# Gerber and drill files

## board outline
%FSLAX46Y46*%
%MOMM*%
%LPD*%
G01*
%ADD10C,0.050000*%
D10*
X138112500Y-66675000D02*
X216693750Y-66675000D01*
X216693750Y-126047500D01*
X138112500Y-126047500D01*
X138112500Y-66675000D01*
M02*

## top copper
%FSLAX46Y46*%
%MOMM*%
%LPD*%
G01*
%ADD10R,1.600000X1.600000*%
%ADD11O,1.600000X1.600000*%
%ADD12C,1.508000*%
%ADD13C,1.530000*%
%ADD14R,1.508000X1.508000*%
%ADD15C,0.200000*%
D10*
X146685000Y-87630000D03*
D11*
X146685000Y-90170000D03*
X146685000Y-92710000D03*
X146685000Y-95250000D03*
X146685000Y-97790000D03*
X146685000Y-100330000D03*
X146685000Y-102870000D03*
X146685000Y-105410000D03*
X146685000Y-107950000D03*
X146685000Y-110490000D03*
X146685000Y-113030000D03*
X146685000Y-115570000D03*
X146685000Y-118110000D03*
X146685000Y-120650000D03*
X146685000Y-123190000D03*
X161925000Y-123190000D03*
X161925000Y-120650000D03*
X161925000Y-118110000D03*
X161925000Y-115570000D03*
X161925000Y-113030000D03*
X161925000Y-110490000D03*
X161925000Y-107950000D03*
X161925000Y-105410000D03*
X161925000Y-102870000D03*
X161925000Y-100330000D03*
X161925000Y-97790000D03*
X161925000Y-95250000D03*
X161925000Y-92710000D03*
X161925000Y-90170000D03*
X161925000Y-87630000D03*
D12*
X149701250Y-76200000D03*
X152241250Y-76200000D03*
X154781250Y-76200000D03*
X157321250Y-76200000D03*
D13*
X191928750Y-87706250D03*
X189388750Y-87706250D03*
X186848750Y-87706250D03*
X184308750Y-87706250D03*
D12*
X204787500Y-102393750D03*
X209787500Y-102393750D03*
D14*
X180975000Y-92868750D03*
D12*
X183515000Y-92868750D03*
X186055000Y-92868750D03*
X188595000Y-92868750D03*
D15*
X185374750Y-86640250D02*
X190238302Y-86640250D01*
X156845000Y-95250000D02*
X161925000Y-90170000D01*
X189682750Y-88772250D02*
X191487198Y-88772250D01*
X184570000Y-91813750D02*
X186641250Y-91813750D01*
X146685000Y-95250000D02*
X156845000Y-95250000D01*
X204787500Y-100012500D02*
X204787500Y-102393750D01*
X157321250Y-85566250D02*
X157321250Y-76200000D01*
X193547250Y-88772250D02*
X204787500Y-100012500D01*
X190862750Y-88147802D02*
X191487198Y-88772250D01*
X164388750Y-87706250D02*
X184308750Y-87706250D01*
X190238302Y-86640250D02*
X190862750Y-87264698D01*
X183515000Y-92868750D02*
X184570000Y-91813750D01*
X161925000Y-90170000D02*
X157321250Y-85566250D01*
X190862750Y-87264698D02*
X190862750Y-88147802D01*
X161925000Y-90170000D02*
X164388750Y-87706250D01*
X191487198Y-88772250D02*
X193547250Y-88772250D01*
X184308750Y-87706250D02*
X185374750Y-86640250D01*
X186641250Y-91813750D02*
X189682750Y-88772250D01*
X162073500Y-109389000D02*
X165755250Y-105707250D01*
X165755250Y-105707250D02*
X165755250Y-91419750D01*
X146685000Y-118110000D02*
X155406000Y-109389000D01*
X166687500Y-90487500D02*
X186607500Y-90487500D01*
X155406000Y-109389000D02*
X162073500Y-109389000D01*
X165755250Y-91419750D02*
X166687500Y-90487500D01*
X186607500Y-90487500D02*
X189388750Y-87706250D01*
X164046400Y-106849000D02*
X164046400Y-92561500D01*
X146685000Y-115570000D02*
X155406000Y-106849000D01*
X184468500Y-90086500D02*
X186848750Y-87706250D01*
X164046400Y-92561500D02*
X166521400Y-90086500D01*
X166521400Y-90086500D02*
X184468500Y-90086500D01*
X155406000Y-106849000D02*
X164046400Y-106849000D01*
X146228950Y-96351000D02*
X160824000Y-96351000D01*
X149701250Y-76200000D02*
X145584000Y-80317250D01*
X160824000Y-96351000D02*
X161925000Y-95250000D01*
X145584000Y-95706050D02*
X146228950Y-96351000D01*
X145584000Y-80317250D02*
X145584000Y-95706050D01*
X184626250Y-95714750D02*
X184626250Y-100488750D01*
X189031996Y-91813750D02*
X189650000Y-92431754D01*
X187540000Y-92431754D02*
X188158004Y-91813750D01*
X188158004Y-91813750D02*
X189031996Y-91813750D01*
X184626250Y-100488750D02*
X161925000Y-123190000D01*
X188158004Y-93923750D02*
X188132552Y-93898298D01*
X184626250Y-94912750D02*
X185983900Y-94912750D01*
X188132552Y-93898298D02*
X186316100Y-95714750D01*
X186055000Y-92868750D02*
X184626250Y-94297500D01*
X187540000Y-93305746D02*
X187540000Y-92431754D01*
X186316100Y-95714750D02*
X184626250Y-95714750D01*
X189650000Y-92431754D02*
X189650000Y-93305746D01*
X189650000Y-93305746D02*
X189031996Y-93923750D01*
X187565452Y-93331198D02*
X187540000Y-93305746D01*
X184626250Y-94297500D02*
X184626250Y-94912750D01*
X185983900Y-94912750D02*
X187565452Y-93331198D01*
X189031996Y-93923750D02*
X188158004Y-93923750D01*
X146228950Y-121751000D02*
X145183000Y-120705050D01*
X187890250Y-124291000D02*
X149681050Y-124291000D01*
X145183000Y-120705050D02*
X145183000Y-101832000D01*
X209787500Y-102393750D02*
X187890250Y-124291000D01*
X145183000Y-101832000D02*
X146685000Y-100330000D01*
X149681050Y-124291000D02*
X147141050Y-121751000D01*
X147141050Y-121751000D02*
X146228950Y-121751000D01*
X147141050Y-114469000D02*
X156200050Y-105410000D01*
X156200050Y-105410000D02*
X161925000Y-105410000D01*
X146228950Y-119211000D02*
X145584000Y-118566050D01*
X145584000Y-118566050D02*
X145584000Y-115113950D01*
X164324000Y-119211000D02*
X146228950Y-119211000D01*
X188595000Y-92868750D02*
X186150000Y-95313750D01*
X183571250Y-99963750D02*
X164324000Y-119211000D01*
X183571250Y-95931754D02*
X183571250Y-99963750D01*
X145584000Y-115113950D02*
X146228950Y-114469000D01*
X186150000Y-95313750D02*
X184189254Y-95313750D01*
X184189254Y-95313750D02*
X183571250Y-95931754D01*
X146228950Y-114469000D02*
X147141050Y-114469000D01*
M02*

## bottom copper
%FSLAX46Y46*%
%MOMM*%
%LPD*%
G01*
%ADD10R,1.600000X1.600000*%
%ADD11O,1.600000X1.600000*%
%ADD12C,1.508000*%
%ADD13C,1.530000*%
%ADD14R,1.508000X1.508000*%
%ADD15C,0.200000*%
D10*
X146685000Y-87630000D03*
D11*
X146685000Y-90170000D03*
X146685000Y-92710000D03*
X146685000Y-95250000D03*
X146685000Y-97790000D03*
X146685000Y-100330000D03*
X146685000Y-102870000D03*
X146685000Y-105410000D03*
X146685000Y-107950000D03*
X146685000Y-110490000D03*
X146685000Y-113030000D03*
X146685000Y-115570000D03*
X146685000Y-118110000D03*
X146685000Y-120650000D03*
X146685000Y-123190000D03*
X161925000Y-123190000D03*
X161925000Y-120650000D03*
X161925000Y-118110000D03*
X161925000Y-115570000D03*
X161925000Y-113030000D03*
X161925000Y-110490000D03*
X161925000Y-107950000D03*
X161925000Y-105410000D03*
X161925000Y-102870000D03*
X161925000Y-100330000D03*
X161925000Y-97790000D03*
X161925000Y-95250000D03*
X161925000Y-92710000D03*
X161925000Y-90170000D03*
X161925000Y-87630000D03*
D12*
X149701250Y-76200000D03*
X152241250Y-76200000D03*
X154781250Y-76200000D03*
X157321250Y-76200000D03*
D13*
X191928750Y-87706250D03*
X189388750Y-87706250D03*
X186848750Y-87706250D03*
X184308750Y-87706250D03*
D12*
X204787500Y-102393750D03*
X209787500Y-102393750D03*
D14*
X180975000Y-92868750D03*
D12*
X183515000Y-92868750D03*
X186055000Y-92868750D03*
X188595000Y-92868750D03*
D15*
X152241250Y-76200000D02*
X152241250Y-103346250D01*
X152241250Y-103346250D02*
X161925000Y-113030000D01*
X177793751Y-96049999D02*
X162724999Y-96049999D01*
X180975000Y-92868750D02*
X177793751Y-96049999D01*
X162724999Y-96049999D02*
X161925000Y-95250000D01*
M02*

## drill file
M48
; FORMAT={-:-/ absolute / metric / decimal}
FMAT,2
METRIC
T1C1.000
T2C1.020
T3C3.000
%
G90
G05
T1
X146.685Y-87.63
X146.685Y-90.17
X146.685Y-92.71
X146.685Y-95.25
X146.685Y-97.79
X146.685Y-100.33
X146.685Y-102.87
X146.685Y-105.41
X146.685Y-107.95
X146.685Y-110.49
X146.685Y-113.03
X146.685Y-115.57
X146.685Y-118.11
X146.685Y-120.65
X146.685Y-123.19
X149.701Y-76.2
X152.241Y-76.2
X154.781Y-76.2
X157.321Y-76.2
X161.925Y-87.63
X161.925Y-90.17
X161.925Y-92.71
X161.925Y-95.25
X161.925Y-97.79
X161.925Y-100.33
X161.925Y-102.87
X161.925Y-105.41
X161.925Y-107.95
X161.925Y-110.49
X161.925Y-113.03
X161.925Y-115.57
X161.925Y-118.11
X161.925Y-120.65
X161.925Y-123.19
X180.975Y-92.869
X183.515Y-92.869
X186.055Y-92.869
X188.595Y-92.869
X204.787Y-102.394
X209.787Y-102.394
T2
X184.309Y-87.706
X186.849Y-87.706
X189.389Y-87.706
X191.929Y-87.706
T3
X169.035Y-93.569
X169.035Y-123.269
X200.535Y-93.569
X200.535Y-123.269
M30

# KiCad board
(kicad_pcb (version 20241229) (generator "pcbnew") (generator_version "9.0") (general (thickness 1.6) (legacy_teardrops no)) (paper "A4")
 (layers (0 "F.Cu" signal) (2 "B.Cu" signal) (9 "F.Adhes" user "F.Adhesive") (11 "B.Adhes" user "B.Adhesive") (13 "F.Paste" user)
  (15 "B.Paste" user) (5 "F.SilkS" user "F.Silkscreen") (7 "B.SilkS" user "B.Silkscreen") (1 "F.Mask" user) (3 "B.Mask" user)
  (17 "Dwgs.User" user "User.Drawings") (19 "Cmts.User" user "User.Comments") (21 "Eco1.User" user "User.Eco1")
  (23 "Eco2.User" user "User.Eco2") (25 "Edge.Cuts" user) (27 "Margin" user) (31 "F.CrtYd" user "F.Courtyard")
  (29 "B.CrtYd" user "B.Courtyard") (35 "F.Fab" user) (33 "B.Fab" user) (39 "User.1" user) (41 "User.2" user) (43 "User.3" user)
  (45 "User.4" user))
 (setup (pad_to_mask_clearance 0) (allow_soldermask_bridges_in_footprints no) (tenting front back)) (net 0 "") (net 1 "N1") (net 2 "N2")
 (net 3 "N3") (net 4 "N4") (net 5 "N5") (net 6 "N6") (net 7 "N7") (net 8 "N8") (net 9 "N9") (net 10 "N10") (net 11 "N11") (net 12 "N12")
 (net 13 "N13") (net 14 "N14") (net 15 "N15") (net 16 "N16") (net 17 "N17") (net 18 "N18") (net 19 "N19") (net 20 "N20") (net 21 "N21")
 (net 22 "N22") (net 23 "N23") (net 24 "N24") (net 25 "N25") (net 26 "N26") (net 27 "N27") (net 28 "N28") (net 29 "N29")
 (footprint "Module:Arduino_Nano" (layer "F.Cu") (at 146.685 87.63)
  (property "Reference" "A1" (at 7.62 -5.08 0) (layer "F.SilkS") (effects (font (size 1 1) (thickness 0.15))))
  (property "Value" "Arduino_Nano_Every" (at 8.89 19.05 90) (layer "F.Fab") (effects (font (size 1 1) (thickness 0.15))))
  (pad "1" thru_hole rect (at 0 0) (size 1.6 1.6) (drill 1) (layers "*.Cu" "*.Mask") (remove_unused_layers no) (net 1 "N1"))
  (pad "2" thru_hole oval (at 0 2.54) (size 1.6 1.6) (drill 1) (layers "*.Cu" "*.Mask") (remove_unused_layers no) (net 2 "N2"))
  (pad "3" thru_hole oval (at 0 5.08) (size 1.6 1.6) (drill 1) (layers "*.Cu" "*.Mask") (remove_unused_layers no) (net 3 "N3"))
  (pad "4" thru_hole oval (at 0 7.62) (size 1.6 1.6) (drill 1) (layers "*.Cu" "*.Mask") (remove_unused_layers no) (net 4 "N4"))
  (pad "5" thru_hole oval (at 0 10.16) (size 1.6 1.6) (drill 1) (layers "*.Cu" "*.Mask") (remove_unused_layers no) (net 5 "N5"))
  (pad "6" thru_hole oval (at 0 12.7) (size 1.6 1.6) (drill 1) (layers "*.Cu" "*.Mask") (remove_unused_layers no) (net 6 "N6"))
  (pad "7" thru_hole oval (at 0 15.24) (size 1.6 1.6) (drill 1) (layers "*.Cu" "*.Mask") (remove_unused_layers no) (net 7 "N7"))
  (pad "8" thru_hole oval (at 0 17.78) (size 1.6 1.6) (drill 1) (layers "*.Cu" "*.Mask") (remove_unused_layers no) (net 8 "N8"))
  (pad "9" thru_hole oval (at 0 20.32) (size 1.6 1.6) (drill 1) (layers "*.Cu" "*.Mask") (remove_unused_layers no) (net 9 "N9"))
  (pad "10" thru_hole oval (at 0 22.86) (size 1.6 1.6) (drill 1) (layers "*.Cu" "*.Mask") (remove_unused_layers no) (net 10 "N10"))
  (pad "11" thru_hole oval (at 0 25.4) (size 1.6 1.6) (drill 1) (layers "*.Cu" "*.Mask") (remove_unused_layers no) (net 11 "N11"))
  (pad "12" thru_hole oval (at 0 27.94) (size 1.6 1.6) (drill 1) (layers "*.Cu" "*.Mask") (remove_unused_layers no) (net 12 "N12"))
  (pad "13" thru_hole oval (at 0 30.48) (size 1.6 1.6) (drill 1) (layers "*.Cu" "*.Mask") (remove_unused_layers no) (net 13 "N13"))
  (pad "14" thru_hole oval (at 0 33.02) (size 1.6 1.6) (drill 1) (layers "*.Cu" "*.Mask") (remove_unused_layers no) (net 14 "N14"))
  (pad "15" thru_hole oval (at 0 35.56) (size 1.6 1.6) (drill 1) (layers "*.Cu" "*.Mask") (remove_unused_layers no) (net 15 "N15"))
  (pad "16" thru_hole oval (at 15.24 35.56) (size 1.6 1.6) (drill 1) (layers "*.Cu" "*.Mask") (remove_unused_layers no) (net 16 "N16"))
  (pad "17" thru_hole oval (at 15.24 33.02) (size 1.6 1.6) (drill 1) (layers "*.Cu" "*.Mask") (remove_unused_layers no) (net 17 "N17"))
  (pad "18" thru_hole oval (at 15.24 30.48) (size 1.6 1.6) (drill 1) (layers "*.Cu" "*.Mask") (remove_unused_layers no) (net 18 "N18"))
  (pad "19" thru_hole oval (at 15.24 27.94) (size 1.6 1.6) (drill 1) (layers "*.Cu" "*.Mask") (remove_unused_layers no) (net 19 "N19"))
  (pad "20" thru_hole oval (at 15.24 25.4) (size 1.6 1.6) (drill 1) (layers "*.Cu" "*.Mask") (remove_unused_layers no) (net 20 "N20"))
  (pad "21" thru_hole oval (at 15.24 22.86) (size 1.6 1.6) (drill 1) (layers "*.Cu" "*.Mask") (remove_unused_layers no) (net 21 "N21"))
  (pad "22" thru_hole oval (at 15.24 20.32) (size 1.6 1.6) (drill 1) (layers "*.Cu" "*.Mask") (remove_unused_layers no) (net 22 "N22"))
  (pad "23" thru_hole oval (at 15.24 17.78) (size 1.6 1.6) (drill 1) (layers "*.Cu" "*.Mask") (remove_unused_layers no) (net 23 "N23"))
  (pad "24" thru_hole oval (at 15.24 15.24) (size 1.6 1.6) (drill 1) (layers "*.Cu" "*.Mask") (remove_unused_layers no) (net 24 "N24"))
  (pad "25" thru_hole oval (at 15.24 12.7) (size 1.6 1.6) (drill 1) (layers "*.Cu" "*.Mask") (remove_unused_layers no) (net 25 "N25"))
  (pad "26" thru_hole oval (at 15.24 10.16) (size 1.6 1.6) (drill 1) (layers "*.Cu" "*.Mask") (remove_unused_layers no) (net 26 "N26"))
  (pad "27" thru_hole oval (at 15.24 7.62) (size 1.6 1.6) (drill 1) (layers "*.Cu" "*.Mask") (remove_unused_layers no) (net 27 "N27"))
  (pad "28" thru_hole oval (at 15.24 5.08) (size 1.6 1.6) (drill 1) (layers "*.Cu" "*.Mask") (remove_unused_layers no) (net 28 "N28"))
  (pad "29" thru_hole oval (at 15.24 2.54) (size 1.6 1.6) (drill 1) (layers "*.Cu" "*.Mask") (remove_unused_layers no) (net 4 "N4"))
  (pad "30" thru_hole oval (at 15.24 0) (size 1.6 1.6) (drill 1) (layers "*.Cu" "*.Mask") (remove_unused_layers no) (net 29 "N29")))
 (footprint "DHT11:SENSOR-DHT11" (layer "F.Cu") (at 153.51125 76.2)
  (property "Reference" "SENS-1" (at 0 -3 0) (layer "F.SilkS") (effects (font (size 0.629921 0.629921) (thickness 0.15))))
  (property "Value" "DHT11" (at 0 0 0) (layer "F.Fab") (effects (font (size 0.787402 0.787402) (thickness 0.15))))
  (pad "P$1" thru_hole circle (at -3.81 0) (size 1.508 1.508) (drill 1) (layers "*.Cu" "*.Mask") (remove_unused_layers no) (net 27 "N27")
   (solder_mask_margin 0.102))
  (pad "P$2" thru_hole circle (at -1.27 0) (size 1.508 1.508) (drill 1) (layers "*.Cu" "*.Mask") (remove_unused_layers no) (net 20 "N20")
   (solder_mask_margin 0.102))
  (pad "P$3" thru_hole circle (at 1.27 0) (size 1.508 1.508) (drill 1) (layers "*.Cu" "*.Mask") (remove_unused_layers no)
   (solder_mask_margin 0.102))
  (pad "P$4" thru_hole circle (at 3.81 0) (size 1.508 1.508) (drill 1) (layers "*.Cu" "*.Mask") (remove_unused_layers no) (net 4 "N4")
   (solder_mask_margin 0.102)))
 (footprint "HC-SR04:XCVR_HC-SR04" (layer "F.Cu") (at 188.11875 87.70625 180)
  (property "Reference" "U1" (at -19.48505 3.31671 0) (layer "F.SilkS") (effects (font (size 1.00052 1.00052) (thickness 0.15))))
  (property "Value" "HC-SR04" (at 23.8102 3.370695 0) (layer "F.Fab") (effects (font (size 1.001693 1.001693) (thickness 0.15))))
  (pad "1" thru_hole circle (at -3.81 0 180) (size 1.53 1.53) (drill 1.02) (layers "*.Cu" "*.Mask") (remove_unused_layers no) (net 27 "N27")
   (solder_mask_margin 0.102))
  (pad "2" thru_hole circle (at -1.27 0 180) (size 1.53 1.53) (drill 1.02) (layers "*.Cu" "*.Mask") (remove_unused_layers no) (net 13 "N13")
   (solder_mask_margin 0.102))
  (pad "3" thru_hole circle (at 1.27 0 180) (size 1.53 1.53) (drill 1.02) (layers "*.Cu" "*.Mask") (remove_unused_layers no) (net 12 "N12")
   (solder_mask_margin 0.102))
  (pad "4" thru_hole circle (at 3.81 0 180) (size 1.53 1.53) (drill 1.02) (layers "*.Cu" "*.Mask") (remove_unused_layers no) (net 4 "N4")
   (solder_mask_margin 0.102)))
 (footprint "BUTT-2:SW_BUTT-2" (layer "F.Cu") (at 207.2875 102.39375)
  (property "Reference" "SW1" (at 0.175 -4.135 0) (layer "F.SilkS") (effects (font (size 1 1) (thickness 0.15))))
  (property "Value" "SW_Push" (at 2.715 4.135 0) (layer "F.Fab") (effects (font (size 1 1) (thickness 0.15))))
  (pad "1" thru_hole circle (at -2.5 0) (size 1.508 1.508) (drill 1) (layers "*.Cu" "*.Mask") (remove_unused_layers no) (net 4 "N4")
   (solder_mask_margin 0.102))
  (pad "2" thru_hole circle (at 2.5 0) (size 1.508 1.508) (drill 1) (layers "*.Cu" "*.Mask") (remove_unused_layers no) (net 6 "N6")
   (solder_mask_margin 0.102)))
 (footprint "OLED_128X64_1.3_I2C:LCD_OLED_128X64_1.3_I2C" (layer "F.Cu") (at 184.785 108.41875)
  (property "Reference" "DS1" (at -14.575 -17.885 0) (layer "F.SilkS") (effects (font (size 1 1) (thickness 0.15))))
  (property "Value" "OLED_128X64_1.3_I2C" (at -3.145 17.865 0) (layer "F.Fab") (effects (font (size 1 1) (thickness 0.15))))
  (pad "" np_thru_hole circle (at -15.75 -14.85) (size 3 3) (drill 3) (layers "*.Cu" "*.Mask"))
  (pad "" np_thru_hole circle (at -15.75 14.85) (size 3 3) (drill 3) (layers "*.Cu" "*.Mask"))
  (pad "" np_thru_hole circle (at 15.75 -14.85) (size 3 3) (drill 3) (layers "*.Cu" "*.Mask"))
  (pad "" np_thru_hole circle (at 15.75 14.85) (size 3 3) (drill 3) (layers "*.Cu" "*.Mask"))
  (pad "1" thru_hole rect (at -3.81 -15.55) (size 1.508 1.508) (drill 1) (layers "*.Cu" "*.Mask") (remove_unused_layers no) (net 27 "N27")
   (solder_mask_margin 0.102))
  (pad "2" thru_hole circle (at -1.27 -15.55) (size 1.508 1.508) (drill 1) (layers "*.Cu" "*.Mask") (remove_unused_layers no) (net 4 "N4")
   (solder_mask_margin 0.102))
  (pad "3" thru_hole circle (at 1.27 -15.55) (size 1.508 1.508) (drill 1) (layers "*.Cu" "*.Mask") (remove_unused_layers no) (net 16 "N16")
   (solder_mask_margin 0.102))
  (pad "4" thru_hole circle (at 3.81 -15.55) (size 1.508 1.508) (drill 1) (layers "*.Cu" "*.Mask") (remove_unused_layers no) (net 23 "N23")
   (solder_mask_margin 0.102)))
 (gr_rect (start 138.1125 66.675) (end 216.69375 126.0475) (stroke (width 0.05) (type default)) (fill no) (layer "Edge.Cuts"))
 (segment (start 185.37475 86.64025) (end 190.238302 86.64025) (width 0.2) (layer "F.Cu") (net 4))
 (segment (start 156.845 95.25) (end 161.925 90.17) (width 0.2) (layer "F.Cu") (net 4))
 (segment (start 189.68275 88.77225) (end 191.487198 88.77225) (width 0.2) (layer "F.Cu") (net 4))
 (segment (start 184.57 91.81375) (end 186.64125 91.81375) (width 0.2) (layer "F.Cu") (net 4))
 (segment (start 146.685 95.25) (end 156.845 95.25) (width 0.2) (layer "F.Cu") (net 4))
 (segment (start 204.7875 100.0125) (end 204.7875 102.39375) (width 0.2) (layer "F.Cu") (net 4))
 (segment (start 157.32125 85.56625) (end 157.32125 76.2) (width 0.2) (layer "F.Cu") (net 4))
 (segment (start 193.54725 88.77225) (end 204.7875 100.0125) (width 0.2) (layer "F.Cu") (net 4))
 (segment (start 190.86275 88.147802) (end 191.487198 88.77225) (width 0.2) (layer "F.Cu") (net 4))
 (segment (start 164.38875 87.70625) (end 184.30875 87.70625) (width 0.2) (layer "F.Cu") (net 4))
 (segment (start 190.238302 86.64025) (end 190.86275 87.264698) (width 0.2) (layer "F.Cu") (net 4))
 (segment (start 183.515 92.86875) (end 184.57 91.81375) (width 0.2) (layer "F.Cu") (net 4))
 (segment (start 161.925 90.17) (end 157.32125 85.56625) (width 0.2) (layer "F.Cu") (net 4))
 (segment (start 190.86275 87.264698) (end 190.86275 88.147802) (width 0.2) (layer "F.Cu") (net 4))
 (segment (start 161.925 90.17) (end 164.38875 87.70625) (width 0.2) (layer "F.Cu") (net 4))
 (segment (start 191.487198 88.77225) (end 193.54725 88.77225) (width 0.2) (layer "F.Cu") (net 4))
 (segment (start 184.30875 87.70625) (end 185.37475 86.64025) (width 0.2) (layer "F.Cu") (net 4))
 (segment (start 186.64125 91.81375) (end 189.68275 88.77225) (width 0.2) (layer "F.Cu") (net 4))
 (segment (start 162.0735 109.389) (end 165.75525 105.70725) (width 0.2) (layer "F.Cu") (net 13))
 (segment (start 165.75525 105.70725) (end 165.75525 91.41975) (width 0.2) (layer "F.Cu") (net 13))
 (segment (start 146.685 118.11) (end 155.406 109.389) (width 0.2) (layer "F.Cu") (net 13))
 (segment (start 166.6875 90.4875) (end 186.6075 90.4875) (width 0.2) (layer "F.Cu") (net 13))
 (segment (start 155.406 109.389) (end 162.0735 109.389) (width 0.2) (layer "F.Cu") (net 13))
 (segment (start 165.75525 91.41975) (end 166.6875 90.4875) (width 0.2) (layer "F.Cu") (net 13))
 (segment (start 186.6075 90.4875) (end 189.38875 87.70625) (width 0.2) (layer "F.Cu") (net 13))
 (segment (start 164.0464 106.849) (end 164.0464 92.5615) (width 0.2) (layer "F.Cu") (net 12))
 (segment (start 146.685 115.57) (end 155.406 106.849) (width 0.2) (layer "F.Cu") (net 12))
 (segment (start 184.4685 90.0865) (end 186.84875 87.70625) (width 0.2) (layer "F.Cu") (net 12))
 (segment (start 164.0464 92.5615) (end 166.5214 90.0865) (width 0.2) (layer "F.Cu") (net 12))
 (segment (start 166.5214 90.0865) (end 184.4685 90.0865) (width 0.2) (layer "F.Cu") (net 12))
 (segment (start 155.406 106.849) (end 164.0464 106.849) (width 0.2) (layer "F.Cu") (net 12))
 (segment (start 152.24125 76.2) (end 152.24125 103.34625) (width 0.2) (layer "B.Cu") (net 20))
 (segment (start 152.24125 103.34625) (end 161.925 113.03) (width 0.2) (layer "B.Cu") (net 20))
 (segment (start 146.22895 96.351) (end 160.824 96.351) (width 0.2) (layer "F.Cu") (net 27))
 (segment (start 149.70125 76.2) (end 145.584 80.31725) (width 0.2) (layer "F.Cu") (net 27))
 (segment (start 160.824 96.351) (end 161.925 95.25) (width 0.2) (layer "F.Cu") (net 27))
 (segment (start 145.584 95.70605) (end 146.22895 96.351) (width 0.2) (layer "F.Cu") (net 27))
 (segment (start 145.584 80.31725) (end 145.584 95.70605) (width 0.2) (layer "F.Cu") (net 27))
 (segment (start 177.793751 96.049999) (end 162.724999 96.049999) (width 0.2) (layer "B.Cu") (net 27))
 (segment (start 180.975 92.86875) (end 177.793751 96.049999) (width 0.2) (layer "B.Cu") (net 27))
 (segment (start 162.724999 96.049999) (end 161.925 95.25) (width 0.2) (layer "B.Cu") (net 27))
 (segment (start 184.62625 95.71475) (end 184.62625 100.48875) (width 0.2) (layer "F.Cu") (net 16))
 (segment (start 189.031996 91.81375) (end 189.65 92.431754) (width 0.2) (layer "F.Cu") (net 16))
 (segment (start 187.54 92.431754) (end 188.158004 91.81375) (width 0.2) (layer "F.Cu") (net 16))
 (segment (start 188.158004 91.81375) (end 189.031996 91.81375) (width 0.2) (layer "F.Cu") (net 16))
 (segment (start 184.62625 100.48875) (end 161.925 123.19) (width 0.2) (layer "F.Cu") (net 16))
 (segment (start 188.158004 93.92375) (end 188.132552 93.898298) (width 0.2) (layer "F.Cu") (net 16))
 (segment (start 184.62625 94.91275) (end 185.9839 94.91275) (width 0.2) (layer "F.Cu") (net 16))
 (segment (start 188.132552 93.898298) (end 186.3161 95.71475) (width 0.2) (layer "F.Cu") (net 16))
 (segment (start 186.055 92.86875) (end 184.62625 94.2975) (width 0.2) (layer "F.Cu") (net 16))
 (segment (start 187.54 93.305746) (end 187.54 92.431754) (width 0.2) (layer "F.Cu") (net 16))
 (segment (start 186.3161 95.71475) (end 184.62625 95.71475) (width 0.2) (layer "F.Cu") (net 16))
 (segment (start 189.65 92.431754) (end 189.65 93.305746) (width 0.2) (layer "F.Cu") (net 16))
 (segment (start 189.65 93.305746) (end 189.031996 93.92375) (width 0.2) (layer "F.Cu") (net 16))
 (segment (start 187.565452 93.331198) (end 187.54 93.305746) (width 0.2) (layer "F.Cu") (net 16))
 (segment (start 184.62625 94.2975) (end 184.62625 94.91275) (width 0.2) (layer "F.Cu") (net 16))
 (segment (start 185.9839 94.91275) (end 187.565452 93.331198) (width 0.2) (layer "F.Cu") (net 16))
 (segment (start 189.031996 93.92375) (end 188.158004 93.92375) (width 0.2) (layer "F.Cu") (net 16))
 (segment (start 146.22895 121.751) (end 145.183 120.70505) (width 0.2) (layer "F.Cu") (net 6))
 (segment (start 187.89025 124.291) (end 149.68105 124.291) (width 0.2) (layer "F.Cu") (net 6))
 (segment (start 145.183 120.70505) (end 145.183 101.832) (width 0.2) (layer "F.Cu") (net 6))
 (segment (start 209.7875 102.39375) (end 187.89025 124.291) (width 0.2) (layer "F.Cu") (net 6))
 (segment (start 145.183 101.832) (end 146.685 100.33) (width 0.2) (layer "F.Cu") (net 6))
 (segment (start 149.68105 124.291) (end 147.14105 121.751) (width 0.2) (layer "F.Cu") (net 6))
 (segment (start 147.14105 121.751) (end 146.22895 121.751) (width 0.2) (layer "F.Cu") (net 6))
 (segment (start 147.14105 114.469) (end 156.20005 105.41) (width 0.2) (layer "F.Cu") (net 23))
 (segment (start 156.20005 105.41) (end 161.925 105.41) (width 0.2) (layer "F.Cu") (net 23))
 (segment (start 146.22895 119.211) (end 145.584 118.56605) (width 0.2) (layer "F.Cu") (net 23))
 (segment (start 145.584 118.56605) (end 145.584 115.11395) (width 0.2) (layer "F.Cu") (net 23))
 (segment (start 164.324 119.211) (end 146.22895 119.211) (width 0.2) (layer "F.Cu") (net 23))
 (segment (start 188.595 92.86875) (end 186.15 95.31375) (width 0.2) (layer "F.Cu") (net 23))
 (segment (start 183.57125 99.96375) (end 164.324 119.211) (width 0.2) (layer "F.Cu") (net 23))
 (segment (start 183.57125 95.931754) (end 183.57125 99.96375) (width 0.2) (layer "F.Cu") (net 23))
 (segment (start 145.584 115.11395) (end 146.22895 114.469) (width 0.2) (layer "F.Cu") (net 23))
 (segment (start 186.15 95.31375) (end 184.189254 95.31375) (width 0.2) (layer "F.Cu") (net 23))
 (segment (start 184.189254 95.31375) (end 183.57125 95.931754) (width 0.2) (layer "F.Cu") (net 23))
 (segment (start 146.22895 114.469) (end 147.14105 114.469) (width 0.2) (layer "F.Cu") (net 23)))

